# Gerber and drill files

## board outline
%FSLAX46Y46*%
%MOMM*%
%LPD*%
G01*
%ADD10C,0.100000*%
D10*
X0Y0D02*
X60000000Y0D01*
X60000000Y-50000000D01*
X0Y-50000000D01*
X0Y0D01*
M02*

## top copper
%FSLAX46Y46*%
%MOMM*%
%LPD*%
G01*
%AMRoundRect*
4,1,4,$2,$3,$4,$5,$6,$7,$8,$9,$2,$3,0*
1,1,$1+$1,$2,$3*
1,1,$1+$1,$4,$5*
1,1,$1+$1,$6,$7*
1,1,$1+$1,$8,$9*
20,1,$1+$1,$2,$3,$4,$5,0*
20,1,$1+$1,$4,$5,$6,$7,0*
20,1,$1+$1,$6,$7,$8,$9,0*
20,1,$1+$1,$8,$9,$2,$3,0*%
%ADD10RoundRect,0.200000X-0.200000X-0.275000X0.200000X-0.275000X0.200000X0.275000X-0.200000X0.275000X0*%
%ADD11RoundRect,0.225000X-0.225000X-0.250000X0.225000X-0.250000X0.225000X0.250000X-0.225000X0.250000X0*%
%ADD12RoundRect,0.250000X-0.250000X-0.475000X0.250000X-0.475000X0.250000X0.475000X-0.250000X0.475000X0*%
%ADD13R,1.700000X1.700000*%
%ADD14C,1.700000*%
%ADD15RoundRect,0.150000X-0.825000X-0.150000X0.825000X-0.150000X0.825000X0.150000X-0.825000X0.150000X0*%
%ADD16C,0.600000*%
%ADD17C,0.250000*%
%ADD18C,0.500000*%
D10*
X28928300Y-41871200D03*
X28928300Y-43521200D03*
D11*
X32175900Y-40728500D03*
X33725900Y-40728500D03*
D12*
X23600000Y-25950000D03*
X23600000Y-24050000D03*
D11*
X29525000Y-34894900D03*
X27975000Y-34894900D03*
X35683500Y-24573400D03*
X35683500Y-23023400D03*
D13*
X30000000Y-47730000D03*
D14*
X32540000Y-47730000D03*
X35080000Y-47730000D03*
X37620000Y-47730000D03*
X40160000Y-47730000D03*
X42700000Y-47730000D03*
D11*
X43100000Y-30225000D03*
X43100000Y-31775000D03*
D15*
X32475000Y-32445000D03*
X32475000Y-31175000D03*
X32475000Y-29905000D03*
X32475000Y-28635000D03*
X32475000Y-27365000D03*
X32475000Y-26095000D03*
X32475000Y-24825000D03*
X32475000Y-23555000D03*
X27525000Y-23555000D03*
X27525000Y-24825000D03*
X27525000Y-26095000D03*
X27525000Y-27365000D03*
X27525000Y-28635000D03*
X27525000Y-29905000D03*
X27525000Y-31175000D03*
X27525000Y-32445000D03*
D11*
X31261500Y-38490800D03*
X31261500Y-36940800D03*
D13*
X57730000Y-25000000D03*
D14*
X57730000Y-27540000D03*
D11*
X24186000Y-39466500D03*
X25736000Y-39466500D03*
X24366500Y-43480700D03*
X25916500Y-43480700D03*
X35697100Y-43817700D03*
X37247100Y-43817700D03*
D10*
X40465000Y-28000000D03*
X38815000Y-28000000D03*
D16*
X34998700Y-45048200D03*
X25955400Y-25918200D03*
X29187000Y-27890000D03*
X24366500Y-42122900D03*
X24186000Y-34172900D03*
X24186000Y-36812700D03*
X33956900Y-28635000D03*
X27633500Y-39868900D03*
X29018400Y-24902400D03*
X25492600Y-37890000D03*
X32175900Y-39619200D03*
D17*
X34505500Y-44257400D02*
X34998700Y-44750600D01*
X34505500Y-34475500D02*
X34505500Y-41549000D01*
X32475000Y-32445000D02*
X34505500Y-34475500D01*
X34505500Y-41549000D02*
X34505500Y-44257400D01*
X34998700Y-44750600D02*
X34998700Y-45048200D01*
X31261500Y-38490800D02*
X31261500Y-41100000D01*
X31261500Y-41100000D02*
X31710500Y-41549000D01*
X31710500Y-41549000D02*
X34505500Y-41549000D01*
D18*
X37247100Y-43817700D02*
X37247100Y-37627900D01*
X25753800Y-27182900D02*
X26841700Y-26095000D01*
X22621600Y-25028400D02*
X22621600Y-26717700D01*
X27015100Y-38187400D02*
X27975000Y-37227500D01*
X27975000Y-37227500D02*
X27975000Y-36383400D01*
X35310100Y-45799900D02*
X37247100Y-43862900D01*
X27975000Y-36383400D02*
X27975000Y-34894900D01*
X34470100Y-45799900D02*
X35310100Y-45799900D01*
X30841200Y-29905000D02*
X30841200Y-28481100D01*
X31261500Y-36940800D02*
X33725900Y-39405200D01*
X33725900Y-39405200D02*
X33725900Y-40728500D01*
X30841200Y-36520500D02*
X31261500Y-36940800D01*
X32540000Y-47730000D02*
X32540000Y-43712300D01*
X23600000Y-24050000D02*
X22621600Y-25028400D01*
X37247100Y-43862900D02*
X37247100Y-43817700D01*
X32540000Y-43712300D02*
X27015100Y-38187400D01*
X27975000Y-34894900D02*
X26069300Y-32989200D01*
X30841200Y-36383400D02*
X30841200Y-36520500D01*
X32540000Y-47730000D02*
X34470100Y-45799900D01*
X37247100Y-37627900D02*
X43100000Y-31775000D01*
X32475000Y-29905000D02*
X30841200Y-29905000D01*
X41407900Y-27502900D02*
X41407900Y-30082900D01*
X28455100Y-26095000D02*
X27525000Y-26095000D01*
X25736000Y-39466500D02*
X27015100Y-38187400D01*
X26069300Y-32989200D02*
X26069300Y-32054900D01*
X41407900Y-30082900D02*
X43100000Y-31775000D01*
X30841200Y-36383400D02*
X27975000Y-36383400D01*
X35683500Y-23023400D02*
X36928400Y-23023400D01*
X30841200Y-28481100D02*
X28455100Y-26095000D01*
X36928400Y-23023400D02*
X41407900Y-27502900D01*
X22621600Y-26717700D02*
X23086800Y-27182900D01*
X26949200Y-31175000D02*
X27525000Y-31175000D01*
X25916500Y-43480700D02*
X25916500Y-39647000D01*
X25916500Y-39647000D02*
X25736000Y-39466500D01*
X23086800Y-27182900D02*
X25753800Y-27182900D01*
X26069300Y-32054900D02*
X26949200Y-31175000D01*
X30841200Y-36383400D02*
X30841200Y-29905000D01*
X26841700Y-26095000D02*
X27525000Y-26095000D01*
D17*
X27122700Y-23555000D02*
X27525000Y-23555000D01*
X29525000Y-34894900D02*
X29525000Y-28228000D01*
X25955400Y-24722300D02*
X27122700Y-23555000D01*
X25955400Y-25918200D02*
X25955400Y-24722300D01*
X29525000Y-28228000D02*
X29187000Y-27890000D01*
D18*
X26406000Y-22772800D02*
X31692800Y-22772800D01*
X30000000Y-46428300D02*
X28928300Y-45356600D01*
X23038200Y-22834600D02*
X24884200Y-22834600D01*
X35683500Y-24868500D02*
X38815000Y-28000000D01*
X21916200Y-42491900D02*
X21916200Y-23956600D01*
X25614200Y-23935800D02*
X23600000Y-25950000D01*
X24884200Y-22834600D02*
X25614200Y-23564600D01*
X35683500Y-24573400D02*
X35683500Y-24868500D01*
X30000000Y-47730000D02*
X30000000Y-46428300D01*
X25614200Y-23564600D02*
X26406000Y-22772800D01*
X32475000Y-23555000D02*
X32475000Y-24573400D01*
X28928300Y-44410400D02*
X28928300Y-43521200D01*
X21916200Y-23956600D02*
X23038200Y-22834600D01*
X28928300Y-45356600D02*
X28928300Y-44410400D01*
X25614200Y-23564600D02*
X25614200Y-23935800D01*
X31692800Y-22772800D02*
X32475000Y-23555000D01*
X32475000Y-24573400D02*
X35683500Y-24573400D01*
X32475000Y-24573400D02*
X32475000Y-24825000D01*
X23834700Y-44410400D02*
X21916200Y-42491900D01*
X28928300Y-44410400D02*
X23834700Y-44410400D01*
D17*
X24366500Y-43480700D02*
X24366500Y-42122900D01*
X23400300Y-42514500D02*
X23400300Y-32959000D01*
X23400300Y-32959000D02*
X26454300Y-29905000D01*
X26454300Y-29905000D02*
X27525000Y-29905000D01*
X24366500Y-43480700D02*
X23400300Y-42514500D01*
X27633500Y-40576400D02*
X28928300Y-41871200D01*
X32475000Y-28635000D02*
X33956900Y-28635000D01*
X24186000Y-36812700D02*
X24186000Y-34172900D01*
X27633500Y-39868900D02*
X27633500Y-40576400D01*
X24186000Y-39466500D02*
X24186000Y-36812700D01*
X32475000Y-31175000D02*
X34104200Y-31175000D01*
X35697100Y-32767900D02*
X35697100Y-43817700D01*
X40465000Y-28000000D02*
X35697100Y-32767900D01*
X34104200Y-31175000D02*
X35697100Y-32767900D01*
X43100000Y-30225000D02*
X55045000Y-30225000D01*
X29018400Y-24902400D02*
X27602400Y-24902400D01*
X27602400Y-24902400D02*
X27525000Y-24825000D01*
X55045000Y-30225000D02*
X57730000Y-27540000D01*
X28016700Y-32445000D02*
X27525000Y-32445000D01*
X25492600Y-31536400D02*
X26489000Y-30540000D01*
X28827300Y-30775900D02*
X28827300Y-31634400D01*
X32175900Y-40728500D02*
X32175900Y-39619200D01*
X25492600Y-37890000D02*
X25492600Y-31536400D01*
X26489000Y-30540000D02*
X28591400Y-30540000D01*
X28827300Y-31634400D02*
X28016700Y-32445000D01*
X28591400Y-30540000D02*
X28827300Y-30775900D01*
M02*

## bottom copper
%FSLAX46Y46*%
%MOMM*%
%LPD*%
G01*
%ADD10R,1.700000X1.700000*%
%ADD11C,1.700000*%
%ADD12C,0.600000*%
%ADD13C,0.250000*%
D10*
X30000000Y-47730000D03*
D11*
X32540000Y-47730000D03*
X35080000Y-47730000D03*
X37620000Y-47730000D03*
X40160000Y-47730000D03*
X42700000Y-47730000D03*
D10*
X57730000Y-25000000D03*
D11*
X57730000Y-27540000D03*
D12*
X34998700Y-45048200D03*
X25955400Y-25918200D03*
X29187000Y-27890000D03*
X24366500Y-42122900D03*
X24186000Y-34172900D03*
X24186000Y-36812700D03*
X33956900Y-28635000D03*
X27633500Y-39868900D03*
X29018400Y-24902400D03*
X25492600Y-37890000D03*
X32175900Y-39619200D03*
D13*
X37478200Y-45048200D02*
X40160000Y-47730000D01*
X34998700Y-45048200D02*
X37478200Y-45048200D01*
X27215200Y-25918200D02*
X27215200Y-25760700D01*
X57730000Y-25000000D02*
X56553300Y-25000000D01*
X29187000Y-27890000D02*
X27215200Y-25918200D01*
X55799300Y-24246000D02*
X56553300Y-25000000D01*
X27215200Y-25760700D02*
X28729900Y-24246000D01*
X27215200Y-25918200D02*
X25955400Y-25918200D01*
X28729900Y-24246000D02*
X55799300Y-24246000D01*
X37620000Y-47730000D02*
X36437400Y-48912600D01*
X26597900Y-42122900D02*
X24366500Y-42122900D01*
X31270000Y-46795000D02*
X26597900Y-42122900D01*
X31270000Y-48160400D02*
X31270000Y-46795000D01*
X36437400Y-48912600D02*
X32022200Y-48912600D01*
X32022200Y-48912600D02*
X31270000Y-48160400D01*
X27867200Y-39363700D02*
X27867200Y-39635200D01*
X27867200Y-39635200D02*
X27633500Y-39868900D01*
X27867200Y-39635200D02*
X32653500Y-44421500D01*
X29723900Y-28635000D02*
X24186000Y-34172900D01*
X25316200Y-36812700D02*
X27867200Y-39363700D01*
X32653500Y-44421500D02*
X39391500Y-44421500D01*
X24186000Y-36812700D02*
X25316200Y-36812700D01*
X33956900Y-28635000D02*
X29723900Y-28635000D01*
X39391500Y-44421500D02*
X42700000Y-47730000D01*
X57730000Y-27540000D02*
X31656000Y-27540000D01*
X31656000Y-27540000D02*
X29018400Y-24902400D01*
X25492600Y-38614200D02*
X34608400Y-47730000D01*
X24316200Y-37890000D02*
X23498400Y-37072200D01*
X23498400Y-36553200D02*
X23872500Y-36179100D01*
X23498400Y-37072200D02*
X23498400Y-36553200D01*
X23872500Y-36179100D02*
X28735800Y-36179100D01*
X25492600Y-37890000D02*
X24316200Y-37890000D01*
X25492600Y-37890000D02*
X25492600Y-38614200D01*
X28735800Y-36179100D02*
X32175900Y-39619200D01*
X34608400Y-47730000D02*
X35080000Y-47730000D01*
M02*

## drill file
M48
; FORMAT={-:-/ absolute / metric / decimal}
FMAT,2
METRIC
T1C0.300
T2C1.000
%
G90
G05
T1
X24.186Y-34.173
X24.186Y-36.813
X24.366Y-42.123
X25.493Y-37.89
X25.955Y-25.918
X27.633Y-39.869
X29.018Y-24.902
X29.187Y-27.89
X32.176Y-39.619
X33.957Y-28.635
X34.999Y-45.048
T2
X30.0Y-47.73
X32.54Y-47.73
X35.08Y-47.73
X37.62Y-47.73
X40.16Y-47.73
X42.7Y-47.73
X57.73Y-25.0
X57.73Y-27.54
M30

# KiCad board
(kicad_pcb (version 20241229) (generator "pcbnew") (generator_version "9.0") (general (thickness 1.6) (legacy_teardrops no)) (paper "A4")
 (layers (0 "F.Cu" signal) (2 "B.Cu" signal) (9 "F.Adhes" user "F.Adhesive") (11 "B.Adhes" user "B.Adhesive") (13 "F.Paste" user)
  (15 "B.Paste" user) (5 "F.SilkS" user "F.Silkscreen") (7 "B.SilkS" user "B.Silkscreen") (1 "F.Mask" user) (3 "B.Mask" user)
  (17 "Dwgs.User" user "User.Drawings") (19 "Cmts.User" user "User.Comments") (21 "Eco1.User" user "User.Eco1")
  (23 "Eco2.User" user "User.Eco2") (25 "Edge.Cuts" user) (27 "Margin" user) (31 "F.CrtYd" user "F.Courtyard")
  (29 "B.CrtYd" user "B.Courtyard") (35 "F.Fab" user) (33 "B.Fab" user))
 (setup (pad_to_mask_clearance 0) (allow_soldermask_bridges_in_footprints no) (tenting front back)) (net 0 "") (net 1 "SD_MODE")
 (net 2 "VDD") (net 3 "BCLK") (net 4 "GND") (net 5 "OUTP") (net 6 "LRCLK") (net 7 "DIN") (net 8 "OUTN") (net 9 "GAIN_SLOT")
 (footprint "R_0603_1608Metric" (layer "F.Cu") (at 28.9283 42.6962 -90)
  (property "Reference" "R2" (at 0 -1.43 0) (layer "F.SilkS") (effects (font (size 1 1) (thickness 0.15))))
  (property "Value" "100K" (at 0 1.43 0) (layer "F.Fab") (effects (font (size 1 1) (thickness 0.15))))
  (pad "1" smd roundrect (at -0.825 0) (size 0.8 0.95) (layers "F.Cu" "F.Mask" "F.Paste") (roundrect_rratio 0.25) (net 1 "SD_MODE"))
  (pad "2" smd roundrect (at 0.825 0) (size 0.8 0.95) (layers "F.Cu" "F.Mask" "F.Paste") (roundrect_rratio 0.25) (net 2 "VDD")))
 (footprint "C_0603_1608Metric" (layer "F.Cu") (at 32.9509 40.7285)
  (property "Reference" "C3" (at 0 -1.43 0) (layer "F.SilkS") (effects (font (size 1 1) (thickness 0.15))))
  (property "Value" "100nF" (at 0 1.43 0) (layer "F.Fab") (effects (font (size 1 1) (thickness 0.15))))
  (pad "1" smd roundrect (at -0.775 0) (size 0.9 0.95) (layers "F.Cu" "F.Mask" "F.Paste") (roundrect_rratio 0.25) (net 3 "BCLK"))
  (pad "2" smd roundrect (at 0.775 0) (size 0.9 0.95) (layers "F.Cu" "F.Mask" "F.Paste") (roundrect_rratio 0.25) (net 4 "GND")))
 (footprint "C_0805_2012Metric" (layer "F.Cu") (at 23.6 25 90)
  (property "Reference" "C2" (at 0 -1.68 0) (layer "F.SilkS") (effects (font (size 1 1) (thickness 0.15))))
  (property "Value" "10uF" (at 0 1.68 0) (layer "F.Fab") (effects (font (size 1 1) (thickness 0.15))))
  (pad "1" smd roundrect (at -0.95 0) (size 1 1.45) (layers "F.Cu" "F.Mask" "F.Paste") (roundrect_rratio 0.25) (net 2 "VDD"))
  (pad "2" smd roundrect (at 0.95 0) (size 1 1.45) (layers "F.Cu" "F.Mask" "F.Paste") (roundrect_rratio 0.25) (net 4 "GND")))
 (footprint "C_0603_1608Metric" (layer "F.Cu") (at 28.75 34.8949 180)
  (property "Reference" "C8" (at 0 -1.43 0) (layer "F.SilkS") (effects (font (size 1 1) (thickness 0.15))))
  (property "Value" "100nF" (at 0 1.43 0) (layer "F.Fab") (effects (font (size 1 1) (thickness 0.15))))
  (pad "1" smd roundrect (at -0.775 0) (size 0.9 0.95) (layers "F.Cu" "F.Mask" "F.Paste") (roundrect_rratio 0.25) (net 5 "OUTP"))
  (pad "2" smd roundrect (at 0.775 0) (size 0.9 0.95) (layers "F.Cu" "F.Mask" "F.Paste") (roundrect_rratio 0.25) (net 4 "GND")))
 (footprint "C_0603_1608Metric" (layer "F.Cu") (at 35.6835 23.7984 90)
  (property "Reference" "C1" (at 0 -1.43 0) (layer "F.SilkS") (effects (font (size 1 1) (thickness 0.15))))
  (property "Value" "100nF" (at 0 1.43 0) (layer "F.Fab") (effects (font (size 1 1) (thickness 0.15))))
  (pad "1" smd roundrect (at -0.775 0) (size 0.9 0.95) (layers "F.Cu" "F.Mask" "F.Paste") (roundrect_rratio 0.25) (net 2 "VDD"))
  (pad "2" smd roundrect (at 0.775 0) (size 0.9 0.95) (layers "F.Cu" "F.Mask" "F.Paste") (roundrect_rratio 0.25) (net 4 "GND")))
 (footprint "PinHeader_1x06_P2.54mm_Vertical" (layer "F.Cu") (at 30 47.73 90)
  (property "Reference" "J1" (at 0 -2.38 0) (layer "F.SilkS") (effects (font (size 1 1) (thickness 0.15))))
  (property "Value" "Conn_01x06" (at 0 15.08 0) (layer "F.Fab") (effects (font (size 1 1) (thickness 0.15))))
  (pad "1" thru_hole rect (at 0 0) (size 1.7 1.7) (drill 1) (layers "*.Cu" "*.Mask") (remove_unused_layers no) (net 2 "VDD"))
  (pad "2" thru_hole circle (at 0 2.54) (size 1.7 1.7) (drill 1) (layers "*.Cu" "*.Mask") (remove_unused_layers no) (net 4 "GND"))
  (pad "3" thru_hole circle (at 0 5.08) (size 1.7 1.7) (drill 1) (layers "*.Cu" "*.Mask") (remove_unused_layers no) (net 3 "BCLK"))
  (pad "4" thru_hole circle (at 0 7.62) (size 1.7 1.7) (drill 1) (layers "*.Cu" "*.Mask") (remove_unused_layers no) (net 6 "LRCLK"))
  (pad "5" thru_hole circle (at 0 10.16) (size 1.7 1.7) (drill 1) (layers "*.Cu" "*.Mask") (remove_unused_layers no) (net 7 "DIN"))
  (pad "6" thru_hole circle (at 0 12.7) (size 1.7 1.7) (drill 1) (layers "*.Cu" "*.Mask") (remove_unused_layers no) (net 1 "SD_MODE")))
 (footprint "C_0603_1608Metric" (layer "F.Cu") (at 43.1 31 -90)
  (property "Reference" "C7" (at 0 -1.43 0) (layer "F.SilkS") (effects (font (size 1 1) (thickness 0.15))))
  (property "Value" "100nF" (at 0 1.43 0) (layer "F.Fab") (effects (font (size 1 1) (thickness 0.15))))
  (pad "1" smd roundrect (at -0.775 0) (size 0.9 0.95) (layers "F.Cu" "F.Mask" "F.Paste") (roundrect_rratio 0.25) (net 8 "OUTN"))
  (pad "2" smd roundrect (at 0.775 0) (size 0.9 0.95) (layers "F.Cu" "F.Mask" "F.Paste") (roundrect_rratio 0.25) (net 4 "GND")))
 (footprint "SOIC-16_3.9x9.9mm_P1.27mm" (layer "F.Cu") (at 30 28 180)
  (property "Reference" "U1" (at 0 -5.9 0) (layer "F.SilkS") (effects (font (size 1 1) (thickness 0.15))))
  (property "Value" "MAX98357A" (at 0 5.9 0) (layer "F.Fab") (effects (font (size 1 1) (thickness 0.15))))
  (pad "1" smd roundrect (at -2.475 -4.445) (size 1.95 0.6) (layers "F.Cu" "F.Mask" "F.Paste") (roundrect_rratio 0.25) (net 7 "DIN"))
  (pad "2" smd roundrect (at -2.475 -3.175) (size 1.95 0.6) (layers "F.Cu" "F.Mask" "F.Paste") (roundrect_rratio 0.25) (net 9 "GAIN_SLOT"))
  (pad "3" smd roundrect (at -2.475 -1.905) (size 1.95 0.6) (layers "F.Cu" "F.Mask" "F.Paste") (roundrect_rratio 0.25) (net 4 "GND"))
  (pad "4" smd roundrect (at -2.475 -0.635) (size 1.95 0.6) (layers "F.Cu" "F.Mask" "F.Paste") (roundrect_rratio 0.25) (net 1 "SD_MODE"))
  (pad "5" smd roundrect (at -2.475 0.635) (size 1.95 0.6) (layers "F.Cu" "F.Mask" "F.Paste") (roundrect_rratio 0.25))
  (pad "6" smd roundrect (at -2.475 1.905) (size 1.95 0.6) (layers "F.Cu" "F.Mask" "F.Paste") (roundrect_rratio 0.25))
  (pad "7" smd roundrect (at -2.475 3.175) (size 1.95 0.6) (layers "F.Cu" "F.Mask" "F.Paste") (roundrect_rratio 0.25) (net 2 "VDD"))
  (pad "8" smd roundrect (at -2.475 4.445) (size 1.95 0.6) (layers "F.Cu" "F.Mask" "F.Paste") (roundrect_rratio 0.25) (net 2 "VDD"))
  (pad "9" smd roundrect (at 2.475 4.445) (size 1.95 0.6) (layers "F.Cu" "F.Mask" "F.Paste") (roundrect_rratio 0.25) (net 5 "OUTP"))
  (pad "10" smd roundrect (at 2.475 3.175) (size 1.95 0.6) (layers "F.Cu" "F.Mask" "F.Paste") (roundrect_rratio 0.25) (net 8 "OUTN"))
  (pad "11" smd roundrect (at 2.475 1.905) (size 1.95 0.6) (layers "F.Cu" "F.Mask" "F.Paste") (roundrect_rratio 0.25) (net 4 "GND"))
  (pad "12" smd roundrect (at 2.475 0.635) (size 1.95 0.6) (layers "F.Cu" "F.Mask" "F.Paste") (roundrect_rratio 0.25))
  (pad "13" smd roundrect (at 2.475 -0.635) (size 1.95 0.6) (layers "F.Cu" "F.Mask" "F.Paste") (roundrect_rratio 0.25))
  (pad "14" smd roundrect (at 2.475 -1.905) (size 1.95 0.6) (layers "F.Cu" "F.Mask" "F.Paste") (roundrect_rratio 0.25) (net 6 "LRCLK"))
  (pad "15" smd roundrect (at 2.475 -3.175) (size 1.95 0.6) (layers "F.Cu" "F.Mask" "F.Paste") (roundrect_rratio 0.25) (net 4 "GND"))
  (pad "16" smd roundrect (at 2.475 -4.445) (size 1.95 0.6) (layers "F.Cu" "F.Mask" "F.Paste") (roundrect_rratio 0.25) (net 3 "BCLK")))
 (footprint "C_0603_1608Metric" (layer "F.Cu") (at 31.2615 37.7158 90)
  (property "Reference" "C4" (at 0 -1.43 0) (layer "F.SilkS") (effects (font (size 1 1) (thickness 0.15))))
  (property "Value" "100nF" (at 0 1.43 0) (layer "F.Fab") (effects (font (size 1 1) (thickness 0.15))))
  (pad "1" smd roundrect (at -0.775 0) (size 0.9 0.95) (layers "F.Cu" "F.Mask" "F.Paste") (roundrect_rratio 0.25) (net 7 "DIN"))
  (pad "2" smd roundrect (at 0.775 0) (size 0.9 0.95) (layers "F.Cu" "F.Mask" "F.Paste") (roundrect_rratio 0.25) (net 4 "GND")))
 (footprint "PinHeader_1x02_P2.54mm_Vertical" (layer "F.Cu") (at 57.73 25)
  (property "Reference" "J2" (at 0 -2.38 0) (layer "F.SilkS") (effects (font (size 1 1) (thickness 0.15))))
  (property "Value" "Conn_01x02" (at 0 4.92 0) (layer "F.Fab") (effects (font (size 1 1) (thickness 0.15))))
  (pad "1" thru_hole rect (at 0 0) (size 1.7 1.7) (drill 1) (layers "*.Cu" "*.Mask") (remove_unused_layers no) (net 5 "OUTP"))
  (pad "2" thru_hole circle (at 0 2.54) (size 1.7 1.7) (drill 1) (layers "*.Cu" "*.Mask") (remove_unused_layers no) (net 8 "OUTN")))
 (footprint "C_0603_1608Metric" (layer "F.Cu") (at 24.961 39.4665)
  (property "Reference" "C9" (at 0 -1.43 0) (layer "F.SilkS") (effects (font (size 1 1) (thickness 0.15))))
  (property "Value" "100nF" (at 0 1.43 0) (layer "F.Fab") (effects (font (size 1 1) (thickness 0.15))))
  (pad "1" smd roundrect (at -0.775 0) (size 0.9 0.95) (layers "F.Cu" "F.Mask" "F.Paste") (roundrect_rratio 0.25) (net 1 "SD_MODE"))
  (pad "2" smd roundrect (at 0.775 0) (size 0.9 0.95) (layers "F.Cu" "F.Mask" "F.Paste") (roundrect_rratio 0.25) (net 4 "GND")))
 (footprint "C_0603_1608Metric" (layer "F.Cu") (at 25.1415 43.4807)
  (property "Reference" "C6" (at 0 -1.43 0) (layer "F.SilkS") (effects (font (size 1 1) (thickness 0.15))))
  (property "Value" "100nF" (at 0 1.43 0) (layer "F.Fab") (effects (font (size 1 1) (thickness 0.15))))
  (pad "1" smd roundrect (at -0.775 0) (size 0.9 0.95) (layers "F.Cu" "F.Mask" "F.Paste") (roundrect_rratio 0.25) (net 6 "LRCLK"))
  (pad "2" smd roundrect (at 0.775 0) (size 0.9 0.95) (layers "F.Cu" "F.Mask" "F.Paste") (roundrect_rratio 0.25) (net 4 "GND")))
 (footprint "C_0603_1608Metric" (layer "F.Cu") (at 36.4721 43.8177)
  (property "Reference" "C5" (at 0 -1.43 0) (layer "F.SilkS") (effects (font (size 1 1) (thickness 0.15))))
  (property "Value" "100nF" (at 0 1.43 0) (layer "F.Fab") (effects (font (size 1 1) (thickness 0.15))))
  (pad "1" smd roundrect (at -0.775 0) (size 0.9 0.95) (layers "F.Cu" "F.Mask" "F.Paste") (roundrect_rratio 0.25) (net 9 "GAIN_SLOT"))
  (pad "2" smd roundrect (at 0.775 0) (size 0.9 0.95) (layers "F.Cu" "F.Mask" "F.Paste") (roundrect_rratio 0.25) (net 4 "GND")))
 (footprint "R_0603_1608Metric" (layer "F.Cu") (at 39.64 28 180)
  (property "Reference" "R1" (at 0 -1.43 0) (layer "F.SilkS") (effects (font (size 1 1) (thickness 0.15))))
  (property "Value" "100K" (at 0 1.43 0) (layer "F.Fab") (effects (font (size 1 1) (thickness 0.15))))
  (pad "1" smd roundrect (at -0.825 0) (size 0.8 0.95) (layers "F.Cu" "F.Mask" "F.Paste") (roundrect_rratio 0.25) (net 9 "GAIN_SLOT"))
  (pad "2" smd roundrect (at 0.825 0) (size 0.8 0.95) (layers "F.Cu" "F.Mask" "F.Paste") (roundrect_rratio 0.25) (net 2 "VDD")))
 (gr_rect (start 0 0) (end 60 50) (stroke (width 0.1) (type solid)) (fill no) (layer "Edge.Cuts"))
 (segment (start 34.5055 44.2574) (end 34.9987 44.7506) (width 0.25) (layer "F.Cu") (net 7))
 (segment (start 34.5055 34.4755) (end 34.5055 41.549) (width 0.25) (layer "F.Cu") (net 7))
 (segment (start 32.475 32.445) (end 34.5055 34.4755) (width 0.25) (layer "F.Cu") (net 7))
 (segment (start 34.5055 41.549) (end 34.5055 44.2574) (width 0.25) (layer "F.Cu") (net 7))
 (segment (start 34.9987 44.7506) (end 34.9987 45.0482) (width 0.25) (layer "F.Cu") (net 7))
 (segment (start 31.2615 38.4908) (end 31.2615 41.1) (width 0.25) (layer "F.Cu") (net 7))
 (segment (start 31.2615 41.1) (end 31.7105 41.549) (width 0.25) (layer "F.Cu") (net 7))
 (segment (start 31.7105 41.549) (end 34.5055 41.549) (width 0.25) (layer "F.Cu") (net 7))
 (via (at 34.9987 45.0482) (size 0.6) (drill 0.3) (layers "F.Cu" "B.Cu") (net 7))
 (segment (start 37.4782 45.0482) (end 40.16 47.73) (width 0.25) (layer "B.Cu") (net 7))
 (segment (start 34.9987 45.0482) (end 37.4782 45.0482) (width 0.25) (layer "B.Cu") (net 7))
 (segment (start 37.2471 43.8177) (end 37.2471 37.6279) (width 0.5) (layer "F.Cu") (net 4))
 (segment (start 25.7538 27.1829) (end 26.8417 26.095) (width 0.5) (layer "F.Cu") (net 4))
 (segment (start 22.6216 25.0284) (end 22.6216 26.7177) (width 0.5) (layer "F.Cu") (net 4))
 (segment (start 27.0151 38.1874) (end 27.975 37.2275) (width 0.5) (layer "F.Cu") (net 4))
 (segment (start 27.975 37.2275) (end 27.975 36.3834) (width 0.5) (layer "F.Cu") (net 4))
 (segment (start 35.3101 45.7999) (end 37.2471 43.8629) (width 0.5) (layer "F.Cu") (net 4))
 (segment (start 27.975 36.3834) (end 27.975 34.8949) (width 0.5) (layer "F.Cu") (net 4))
 (segment (start 34.4701 45.7999) (end 35.3101 45.7999) (width 0.5) (layer "F.Cu") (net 4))
 (segment (start 30.8412 29.905) (end 30.8412 28.4811) (width 0.5) (layer "F.Cu") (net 4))
 (segment (start 31.2615 36.9408) (end 33.7259 39.4052) (width 0.5) (layer "F.Cu") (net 4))
 (segment (start 33.7259 39.4052) (end 33.7259 40.7285) (width 0.5) (layer "F.Cu") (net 4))
 (segment (start 30.8412 36.5205) (end 31.2615 36.9408) (width 0.5) (layer "F.Cu") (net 4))
 (segment (start 32.54 47.73) (end 32.54 43.7123) (width 0.5) (layer "F.Cu") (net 4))
 (segment (start 23.6 24.05) (end 22.6216 25.0284) (width 0.5) (layer "F.Cu") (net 4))
 (segment (start 37.2471 43.8629) (end 37.2471 43.8177) (width 0.5) (layer "F.Cu") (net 4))
 (segment (start 32.54 43.7123) (end 27.0151 38.1874) (width 0.5) (layer "F.Cu") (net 4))
 (segment (start 27.975 34.8949) (end 26.0693 32.9892) (width 0.5) (layer "F.Cu") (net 4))
 (segment (start 30.8412 36.3834) (end 30.8412 36.5205) (width 0.5) (layer "F.Cu") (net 4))
 (segment (start 32.54 47.73) (end 34.4701 45.7999) (width 0.5) (layer "F.Cu") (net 4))
 (segment (start 37.2471 37.6279) (end 43.1 31.775) (width 0.5) (layer "F.Cu") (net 4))
 (segment (start 32.475 29.905) (end 30.8412 29.905) (width 0.5) (layer "F.Cu") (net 4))
 (segment (start 41.4079 27.5029) (end 41.4079 30.0829) (width 0.5) (layer "F.Cu") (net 4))
 (segment (start 28.4551 26.095) (end 27.525 26.095) (width 0.5) (layer "F.Cu") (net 4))
 (segment (start 25.736 39.4665) (end 27.0151 38.1874) (width 0.5) (layer "F.Cu") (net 4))
 (segment (start 26.0693 32.9892) (end 26.0693 32.0549) (width 0.5) (layer "F.Cu") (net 4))
 (segment (start 41.4079 30.0829) (end 43.1 31.775) (width 0.5) (layer "F.Cu") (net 4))
 (segment (start 30.8412 36.3834) (end 27.975 36.3834) (width 0.5) (layer "F.Cu") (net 4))
 (segment (start 35.6835 23.0234) (end 36.9284 23.0234) (width 0.5) (layer "F.Cu") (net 4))
 (segment (start 30.8412 28.4811) (end 28.4551 26.095) (width 0.5) (layer "F.Cu") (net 4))
 (segment (start 36.9284 23.0234) (end 41.4079 27.5029) (width 0.5) (layer "F.Cu") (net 4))
 (segment (start 22.6216 26.7177) (end 23.0868 27.1829) (width 0.5) (layer "F.Cu") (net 4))
 (segment (start 26.9492 31.175) (end 27.525 31.175) (width 0.5) (layer "F.Cu") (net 4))
 (segment (start 25.9165 43.4807) (end 25.9165 39.647) (width 0.5) (layer "F.Cu") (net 4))
 (segment (start 25.9165 39.647) (end 25.736 39.4665) (width 0.5) (layer "F.Cu") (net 4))
 (segment (start 23.0868 27.1829) (end 25.7538 27.1829) (width 0.5) (layer "F.Cu") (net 4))
 (segment (start 26.0693 32.0549) (end 26.9492 31.175) (width 0.5) (layer "F.Cu") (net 4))
 (segment (start 30.8412 36.3834) (end 30.8412 29.905) (width 0.5) (layer "F.Cu") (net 4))
 (segment (start 26.8417 26.095) (end 27.525 26.095) (width 0.5) (layer "F.Cu") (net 4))
 (segment (start 27.1227 23.555) (end 27.525 23.555) (width 0.25) (layer "F.Cu") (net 5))
 (segment (start 29.525 34.8949) (end 29.525 28.228) (width 0.25) (layer "F.Cu") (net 5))
 (segment (start 25.9554 24.7223) (end 27.1227 23.555) (width 0.25) (layer "F.Cu") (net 5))
 (segment (start 25.9554 25.9182) (end 25.9554 24.7223) (width 0.25) (layer "F.Cu") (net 5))
 (segment (start 29.525 28.228) (end 29.187 27.89) (width 0.25) (layer "F.Cu") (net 5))
 (via (at 25.9554 25.9182) (size 0.6) (drill 0.3) (layers "F.Cu" "B.Cu") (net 5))
 (via (at 29.187 27.89) (size 0.6) (drill 0.3) (layers "F.Cu" "B.Cu") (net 5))
 (segment (start 27.2152 25.9182) (end 27.2152 25.7607) (width 0.25) (layer "B.Cu") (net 5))
 (segment (start 57.73 25) (end 56.5533 25) (width 0.25) (layer "B.Cu") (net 5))
 (segment (start 29.187 27.89) (end 27.2152 25.9182) (width 0.25) (layer "B.Cu") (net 5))
 (segment (start 55.7993 24.246) (end 56.5533 25) (width 0.25) (layer "B.Cu") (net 5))
 (segment (start 27.2152 25.7607) (end 28.7299 24.246) (width 0.25) (layer "B.Cu") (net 5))
 (segment (start 27.2152 25.9182) (end 25.9554 25.9182) (width 0.25) (layer "B.Cu") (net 5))
 (segment (start 28.7299 24.246) (end 55.7993 24.246) (width 0.25) (layer "B.Cu") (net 5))
 (segment (start 26.406 22.7728) (end 31.6928 22.7728) (width 0.5) (layer "F.Cu") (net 2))
 (segment (start 30 46.4283) (end 28.9283 45.3566) (width 0.5) (layer "F.Cu") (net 2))
 (segment (start 23.0382 22.8346) (end 24.8842 22.8346) (width 0.5) (layer "F.Cu") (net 2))
 (segment (start 35.6835 24.8685) (end 38.815 28) (width 0.5) (layer "F.Cu") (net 2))
 (segment (start 21.9162 42.4919) (end 21.9162 23.9566) (width 0.5) (layer "F.Cu") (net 2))
 (segment (start 25.6142 23.9358) (end 23.6 25.95) (width 0.5) (layer "F.Cu") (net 2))
 (segment (start 24.8842 22.8346) (end 25.6142 23.5646) (width 0.5) (layer "F.Cu") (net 2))
 (segment (start 35.6835 24.5734) (end 35.6835 24.8685) (width 0.5) (layer "F.Cu") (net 2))
 (segment (start 30 47.73) (end 30 46.4283) (width 0.5) (layer "F.Cu") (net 2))
 (segment (start 25.6142 23.5646) (end 26.406 22.7728) (width 0.5) (layer "F.Cu") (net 2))
 (segment (start 32.475 23.555) (end 32.475 24.5734) (width 0.5) (layer "F.Cu") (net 2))
 (segment (start 28.9283 44.4104) (end 28.9283 43.5212) (width 0.5) (layer "F.Cu") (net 2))
 (segment (start 21.9162 23.9566) (end 23.0382 22.8346) (width 0.5) (layer "F.Cu") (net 2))
 (segment (start 28.9283 45.3566) (end 28.9283 44.4104) (width 0.5) (layer "F.Cu") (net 2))
 (segment (start 25.6142 23.5646) (end 25.6142 23.9358) (width 0.5) (layer "F.Cu") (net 2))
 (segment (start 31.6928 22.7728) (end 32.475 23.555) (width 0.5) (layer "F.Cu") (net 2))
 (segment (start 32.475 24.5734) (end 35.6835 24.5734) (width 0.5) (layer "F.Cu") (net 2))
 (segment (start 32.475 24.5734) (end 32.475 24.825) (width 0.5) (layer "F.Cu") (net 2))
 (segment (start 23.8347 44.4104) (end 21.9162 42.4919) (width 0.5) (layer "F.Cu") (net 2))
 (segment (start 28.9283 44.4104) (end 23.8347 44.4104) (width 0.5) (layer "F.Cu") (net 2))
 (segment (start 24.3665 43.4807) (end 24.3665 42.1229) (width 0.25) (layer "F.Cu") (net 6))
 (segment (start 23.4003 42.5145) (end 23.4003 32.959) (width 0.25) (layer "F.Cu") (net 6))
 (segment (start 23.4003 32.959) (end 26.4543 29.905) (width 0.25) (layer "F.Cu") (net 6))
 (segment (start 26.4543 29.905) (end 27.525 29.905) (width 0.25) (layer "F.Cu") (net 6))
 (segment (start 24.3665 43.4807) (end 23.4003 42.5145) (width 0.25) (layer "F.Cu") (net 6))
 (via (at 24.3665 42.1229) (size 0.6) (drill 0.3) (layers "F.Cu" "B.Cu") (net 6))
 (segment (start 37.62 47.73) (end 36.4374 48.9126) (width 0.25) (layer "B.Cu") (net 6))
 (segment (start 26.5979 42.1229) (end 24.3665 42.1229) (width 0.25) (layer "B.Cu") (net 6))
 (segment (start 31.27 46.795) (end 26.5979 42.1229) (width 0.25) (layer "B.Cu") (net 6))
 (segment (start 31.27 48.1604) (end 31.27 46.795) (width 0.25) (layer "B.Cu") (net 6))
 (segment (start 36.4374 48.9126) (end 32.0222 48.9126) (width 0.25) (layer "B.Cu") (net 6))
 (segment (start 32.0222 48.9126) (end 31.27 48.1604) (width 0.25) (layer "B.Cu") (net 6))
 (segment (start 27.6335 40.5764) (end 28.9283 41.8712) (width 0.25) (layer "F.Cu") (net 1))
 (segment (start 32.475 28.635) (end 33.9569 28.635) (width 0.25) (layer "F.Cu") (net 1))
 (segment (start 24.186 36.8127) (end 24.186 34.1729) (width 0.25) (layer "F.Cu") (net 1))
 (segment (start 27.6335 39.8689) (end 27.6335 40.5764) (width 0.25) (layer "F.Cu") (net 1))
 (segment (start 24.186 39.4665) (end 24.186 36.8127) (width 0.25) (layer "F.Cu") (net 1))
 (via (at 24.186 34.1729) (size 0.6) (drill 0.3) (layers "F.Cu" "B.Cu") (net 1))
 (via (at 24.186 36.8127) (size 0.6) (drill 0.3) (layers "F.Cu" "B.Cu") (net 1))
 (via (at 33.9569 28.635) (size 0.6) (drill 0.3) (layers "F.Cu" "B.Cu") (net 1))
 (via (at 27.6335 39.8689) (size 0.6) (drill 0.3) (layers "F.Cu" "B.Cu") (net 1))
 (segment (start 27.8672 39.3637) (end 27.8672 39.6352) (width 0.25) (layer "B.Cu") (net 1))
 (segment (start 27.8672 39.6352) (end 27.6335 39.8689) (width 0.25) (layer "B.Cu") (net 1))
 (segment (start 27.8672 39.6352) (end 32.6535 44.4215) (width 0.25) (layer "B.Cu") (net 1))
 (segment (start 29.7239 28.635) (end 24.186 34.1729) (width 0.25) (layer "B.Cu") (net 1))
 (segment (start 25.3162 36.8127) (end 27.8672 39.3637) (width 0.25) (layer "B.Cu") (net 1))
 (segment (start 32.6535 44.4215) (end 39.3915 44.4215) (width 0.25) (layer "B.Cu") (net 1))
 (segment (start 24.186 36.8127) (end 25.3162 36.8127) (width 0.25) (layer "B.Cu") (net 1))
 (segment (start 33.9569 28.635) (end 29.7239 28.635) (width 0.25) (layer "B.Cu") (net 1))
 (segment (start 39.3915 44.4215) (end 42.7 47.73) (width 0.25) (layer "B.Cu") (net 1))
 (segment (start 32.475 31.175) (end 34.1042 31.175) (width 0.25) (layer "F.Cu") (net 9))
 (segment (start 35.6971 32.7679) (end 35.6971 43.8177) (width 0.25) (layer "F.Cu") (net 9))
 (segment (start 40.465 28) (end 35.6971 32.7679) (width 0.25) (layer "F.Cu") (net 9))
 (segment (start 34.1042 31.175) (end 35.6971 32.7679) (width 0.25) (layer "F.Cu") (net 9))
 (segment (start 43.1 30.225) (end 55.045 30.225) (width 0.25) (layer "F.Cu") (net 8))
 (segment (start 29.0184 24.9024) (end 27.6024 24.9024) (width 0.25) (layer "F.Cu") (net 8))
 (segment (start 27.6024 24.9024) (end 27.525 24.825) (width 0.25) (layer "F.Cu") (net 8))
 (segment (start 55.045 30.225) (end 57.73 27.54) (width 0.25) (layer "F.Cu") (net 8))
 (via (at 29.0184 24.9024) (size 0.6) (drill 0.3) (layers "F.Cu" "B.Cu") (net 8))
 (segment (start 57.73 27.54) (end 31.656 27.54) (width 0.25) (layer "B.Cu") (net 8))
 (segment (start 31.656 27.54) (end 29.0184 24.9024) (width 0.25) (layer "B.Cu") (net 8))
 (segment (start 28.0167 32.445) (end 27.525 32.445) (width 0.25) (layer "F.Cu") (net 3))
 (segment (start 25.4926 31.5364) (end 26.489 30.54) (width 0.25) (layer "F.Cu") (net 3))
 (segment (start 28.8273 30.7759) (end 28.8273 31.6344) (width 0.25) (layer "F.Cu") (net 3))
 (segment (start 32.1759 40.7285) (end 32.1759 39.6192) (width 0.25) (layer "F.Cu") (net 3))
 (segment (start 25.4926 37.89) (end 25.4926 31.5364) (width 0.25) (layer "F.Cu") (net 3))
 (segment (start 26.489 30.54) (end 28.5914 30.54) (width 0.25) (layer "F.Cu") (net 3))
 (segment (start 28.8273 31.6344) (end 28.0167 32.445) (width 0.25) (layer "F.Cu") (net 3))
 (segment (start 28.5914 30.54) (end 28.8273 30.7759) (width 0.25) (layer "F.Cu") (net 3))
 (via (at 25.4926 37.89) (size 0.6) (drill 0.3) (layers "F.Cu" "B.Cu") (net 3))
 (via (at 32.1759 39.6192) (size 0.6) (drill 0.3) (layers "F.Cu" "B.Cu") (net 3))
 (segment (start 25.4926 38.6142) (end 34.6084 47.73) (width 0.25) (layer "B.Cu") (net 3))
 (segment (start 24.3162 37.89) (end 23.4984 37.0722) (width 0.25) (layer "B.Cu") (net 3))
 (segment (start 23.4984 36.5532) (end 23.8725 36.1791) (width 0.25) (layer "B.Cu") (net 3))
 (segment (start 23.4984 37.0722) (end 23.4984 36.5532) (width 0.25) (layer "B.Cu") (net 3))
 (segment (start 23.8725 36.1791) (end 28.7358 36.1791) (width 0.25) (layer "B.Cu") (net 3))
 (segment (start 25.4926 37.89) (end 24.3162 37.89) (width 0.25) (layer "B.Cu") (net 3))
 (segment (start 25.4926 37.89) (end 25.4926 38.6142) (width 0.25) (layer "B.Cu") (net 3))
 (segment (start 28.7358 36.1791) (end 32.1759 39.6192) (width 0.25) (layer "B.Cu") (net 3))
 (segment (start 34.6084 47.73) (end 35.08 47.73) (width 0.25) (layer "B.Cu") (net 3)))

